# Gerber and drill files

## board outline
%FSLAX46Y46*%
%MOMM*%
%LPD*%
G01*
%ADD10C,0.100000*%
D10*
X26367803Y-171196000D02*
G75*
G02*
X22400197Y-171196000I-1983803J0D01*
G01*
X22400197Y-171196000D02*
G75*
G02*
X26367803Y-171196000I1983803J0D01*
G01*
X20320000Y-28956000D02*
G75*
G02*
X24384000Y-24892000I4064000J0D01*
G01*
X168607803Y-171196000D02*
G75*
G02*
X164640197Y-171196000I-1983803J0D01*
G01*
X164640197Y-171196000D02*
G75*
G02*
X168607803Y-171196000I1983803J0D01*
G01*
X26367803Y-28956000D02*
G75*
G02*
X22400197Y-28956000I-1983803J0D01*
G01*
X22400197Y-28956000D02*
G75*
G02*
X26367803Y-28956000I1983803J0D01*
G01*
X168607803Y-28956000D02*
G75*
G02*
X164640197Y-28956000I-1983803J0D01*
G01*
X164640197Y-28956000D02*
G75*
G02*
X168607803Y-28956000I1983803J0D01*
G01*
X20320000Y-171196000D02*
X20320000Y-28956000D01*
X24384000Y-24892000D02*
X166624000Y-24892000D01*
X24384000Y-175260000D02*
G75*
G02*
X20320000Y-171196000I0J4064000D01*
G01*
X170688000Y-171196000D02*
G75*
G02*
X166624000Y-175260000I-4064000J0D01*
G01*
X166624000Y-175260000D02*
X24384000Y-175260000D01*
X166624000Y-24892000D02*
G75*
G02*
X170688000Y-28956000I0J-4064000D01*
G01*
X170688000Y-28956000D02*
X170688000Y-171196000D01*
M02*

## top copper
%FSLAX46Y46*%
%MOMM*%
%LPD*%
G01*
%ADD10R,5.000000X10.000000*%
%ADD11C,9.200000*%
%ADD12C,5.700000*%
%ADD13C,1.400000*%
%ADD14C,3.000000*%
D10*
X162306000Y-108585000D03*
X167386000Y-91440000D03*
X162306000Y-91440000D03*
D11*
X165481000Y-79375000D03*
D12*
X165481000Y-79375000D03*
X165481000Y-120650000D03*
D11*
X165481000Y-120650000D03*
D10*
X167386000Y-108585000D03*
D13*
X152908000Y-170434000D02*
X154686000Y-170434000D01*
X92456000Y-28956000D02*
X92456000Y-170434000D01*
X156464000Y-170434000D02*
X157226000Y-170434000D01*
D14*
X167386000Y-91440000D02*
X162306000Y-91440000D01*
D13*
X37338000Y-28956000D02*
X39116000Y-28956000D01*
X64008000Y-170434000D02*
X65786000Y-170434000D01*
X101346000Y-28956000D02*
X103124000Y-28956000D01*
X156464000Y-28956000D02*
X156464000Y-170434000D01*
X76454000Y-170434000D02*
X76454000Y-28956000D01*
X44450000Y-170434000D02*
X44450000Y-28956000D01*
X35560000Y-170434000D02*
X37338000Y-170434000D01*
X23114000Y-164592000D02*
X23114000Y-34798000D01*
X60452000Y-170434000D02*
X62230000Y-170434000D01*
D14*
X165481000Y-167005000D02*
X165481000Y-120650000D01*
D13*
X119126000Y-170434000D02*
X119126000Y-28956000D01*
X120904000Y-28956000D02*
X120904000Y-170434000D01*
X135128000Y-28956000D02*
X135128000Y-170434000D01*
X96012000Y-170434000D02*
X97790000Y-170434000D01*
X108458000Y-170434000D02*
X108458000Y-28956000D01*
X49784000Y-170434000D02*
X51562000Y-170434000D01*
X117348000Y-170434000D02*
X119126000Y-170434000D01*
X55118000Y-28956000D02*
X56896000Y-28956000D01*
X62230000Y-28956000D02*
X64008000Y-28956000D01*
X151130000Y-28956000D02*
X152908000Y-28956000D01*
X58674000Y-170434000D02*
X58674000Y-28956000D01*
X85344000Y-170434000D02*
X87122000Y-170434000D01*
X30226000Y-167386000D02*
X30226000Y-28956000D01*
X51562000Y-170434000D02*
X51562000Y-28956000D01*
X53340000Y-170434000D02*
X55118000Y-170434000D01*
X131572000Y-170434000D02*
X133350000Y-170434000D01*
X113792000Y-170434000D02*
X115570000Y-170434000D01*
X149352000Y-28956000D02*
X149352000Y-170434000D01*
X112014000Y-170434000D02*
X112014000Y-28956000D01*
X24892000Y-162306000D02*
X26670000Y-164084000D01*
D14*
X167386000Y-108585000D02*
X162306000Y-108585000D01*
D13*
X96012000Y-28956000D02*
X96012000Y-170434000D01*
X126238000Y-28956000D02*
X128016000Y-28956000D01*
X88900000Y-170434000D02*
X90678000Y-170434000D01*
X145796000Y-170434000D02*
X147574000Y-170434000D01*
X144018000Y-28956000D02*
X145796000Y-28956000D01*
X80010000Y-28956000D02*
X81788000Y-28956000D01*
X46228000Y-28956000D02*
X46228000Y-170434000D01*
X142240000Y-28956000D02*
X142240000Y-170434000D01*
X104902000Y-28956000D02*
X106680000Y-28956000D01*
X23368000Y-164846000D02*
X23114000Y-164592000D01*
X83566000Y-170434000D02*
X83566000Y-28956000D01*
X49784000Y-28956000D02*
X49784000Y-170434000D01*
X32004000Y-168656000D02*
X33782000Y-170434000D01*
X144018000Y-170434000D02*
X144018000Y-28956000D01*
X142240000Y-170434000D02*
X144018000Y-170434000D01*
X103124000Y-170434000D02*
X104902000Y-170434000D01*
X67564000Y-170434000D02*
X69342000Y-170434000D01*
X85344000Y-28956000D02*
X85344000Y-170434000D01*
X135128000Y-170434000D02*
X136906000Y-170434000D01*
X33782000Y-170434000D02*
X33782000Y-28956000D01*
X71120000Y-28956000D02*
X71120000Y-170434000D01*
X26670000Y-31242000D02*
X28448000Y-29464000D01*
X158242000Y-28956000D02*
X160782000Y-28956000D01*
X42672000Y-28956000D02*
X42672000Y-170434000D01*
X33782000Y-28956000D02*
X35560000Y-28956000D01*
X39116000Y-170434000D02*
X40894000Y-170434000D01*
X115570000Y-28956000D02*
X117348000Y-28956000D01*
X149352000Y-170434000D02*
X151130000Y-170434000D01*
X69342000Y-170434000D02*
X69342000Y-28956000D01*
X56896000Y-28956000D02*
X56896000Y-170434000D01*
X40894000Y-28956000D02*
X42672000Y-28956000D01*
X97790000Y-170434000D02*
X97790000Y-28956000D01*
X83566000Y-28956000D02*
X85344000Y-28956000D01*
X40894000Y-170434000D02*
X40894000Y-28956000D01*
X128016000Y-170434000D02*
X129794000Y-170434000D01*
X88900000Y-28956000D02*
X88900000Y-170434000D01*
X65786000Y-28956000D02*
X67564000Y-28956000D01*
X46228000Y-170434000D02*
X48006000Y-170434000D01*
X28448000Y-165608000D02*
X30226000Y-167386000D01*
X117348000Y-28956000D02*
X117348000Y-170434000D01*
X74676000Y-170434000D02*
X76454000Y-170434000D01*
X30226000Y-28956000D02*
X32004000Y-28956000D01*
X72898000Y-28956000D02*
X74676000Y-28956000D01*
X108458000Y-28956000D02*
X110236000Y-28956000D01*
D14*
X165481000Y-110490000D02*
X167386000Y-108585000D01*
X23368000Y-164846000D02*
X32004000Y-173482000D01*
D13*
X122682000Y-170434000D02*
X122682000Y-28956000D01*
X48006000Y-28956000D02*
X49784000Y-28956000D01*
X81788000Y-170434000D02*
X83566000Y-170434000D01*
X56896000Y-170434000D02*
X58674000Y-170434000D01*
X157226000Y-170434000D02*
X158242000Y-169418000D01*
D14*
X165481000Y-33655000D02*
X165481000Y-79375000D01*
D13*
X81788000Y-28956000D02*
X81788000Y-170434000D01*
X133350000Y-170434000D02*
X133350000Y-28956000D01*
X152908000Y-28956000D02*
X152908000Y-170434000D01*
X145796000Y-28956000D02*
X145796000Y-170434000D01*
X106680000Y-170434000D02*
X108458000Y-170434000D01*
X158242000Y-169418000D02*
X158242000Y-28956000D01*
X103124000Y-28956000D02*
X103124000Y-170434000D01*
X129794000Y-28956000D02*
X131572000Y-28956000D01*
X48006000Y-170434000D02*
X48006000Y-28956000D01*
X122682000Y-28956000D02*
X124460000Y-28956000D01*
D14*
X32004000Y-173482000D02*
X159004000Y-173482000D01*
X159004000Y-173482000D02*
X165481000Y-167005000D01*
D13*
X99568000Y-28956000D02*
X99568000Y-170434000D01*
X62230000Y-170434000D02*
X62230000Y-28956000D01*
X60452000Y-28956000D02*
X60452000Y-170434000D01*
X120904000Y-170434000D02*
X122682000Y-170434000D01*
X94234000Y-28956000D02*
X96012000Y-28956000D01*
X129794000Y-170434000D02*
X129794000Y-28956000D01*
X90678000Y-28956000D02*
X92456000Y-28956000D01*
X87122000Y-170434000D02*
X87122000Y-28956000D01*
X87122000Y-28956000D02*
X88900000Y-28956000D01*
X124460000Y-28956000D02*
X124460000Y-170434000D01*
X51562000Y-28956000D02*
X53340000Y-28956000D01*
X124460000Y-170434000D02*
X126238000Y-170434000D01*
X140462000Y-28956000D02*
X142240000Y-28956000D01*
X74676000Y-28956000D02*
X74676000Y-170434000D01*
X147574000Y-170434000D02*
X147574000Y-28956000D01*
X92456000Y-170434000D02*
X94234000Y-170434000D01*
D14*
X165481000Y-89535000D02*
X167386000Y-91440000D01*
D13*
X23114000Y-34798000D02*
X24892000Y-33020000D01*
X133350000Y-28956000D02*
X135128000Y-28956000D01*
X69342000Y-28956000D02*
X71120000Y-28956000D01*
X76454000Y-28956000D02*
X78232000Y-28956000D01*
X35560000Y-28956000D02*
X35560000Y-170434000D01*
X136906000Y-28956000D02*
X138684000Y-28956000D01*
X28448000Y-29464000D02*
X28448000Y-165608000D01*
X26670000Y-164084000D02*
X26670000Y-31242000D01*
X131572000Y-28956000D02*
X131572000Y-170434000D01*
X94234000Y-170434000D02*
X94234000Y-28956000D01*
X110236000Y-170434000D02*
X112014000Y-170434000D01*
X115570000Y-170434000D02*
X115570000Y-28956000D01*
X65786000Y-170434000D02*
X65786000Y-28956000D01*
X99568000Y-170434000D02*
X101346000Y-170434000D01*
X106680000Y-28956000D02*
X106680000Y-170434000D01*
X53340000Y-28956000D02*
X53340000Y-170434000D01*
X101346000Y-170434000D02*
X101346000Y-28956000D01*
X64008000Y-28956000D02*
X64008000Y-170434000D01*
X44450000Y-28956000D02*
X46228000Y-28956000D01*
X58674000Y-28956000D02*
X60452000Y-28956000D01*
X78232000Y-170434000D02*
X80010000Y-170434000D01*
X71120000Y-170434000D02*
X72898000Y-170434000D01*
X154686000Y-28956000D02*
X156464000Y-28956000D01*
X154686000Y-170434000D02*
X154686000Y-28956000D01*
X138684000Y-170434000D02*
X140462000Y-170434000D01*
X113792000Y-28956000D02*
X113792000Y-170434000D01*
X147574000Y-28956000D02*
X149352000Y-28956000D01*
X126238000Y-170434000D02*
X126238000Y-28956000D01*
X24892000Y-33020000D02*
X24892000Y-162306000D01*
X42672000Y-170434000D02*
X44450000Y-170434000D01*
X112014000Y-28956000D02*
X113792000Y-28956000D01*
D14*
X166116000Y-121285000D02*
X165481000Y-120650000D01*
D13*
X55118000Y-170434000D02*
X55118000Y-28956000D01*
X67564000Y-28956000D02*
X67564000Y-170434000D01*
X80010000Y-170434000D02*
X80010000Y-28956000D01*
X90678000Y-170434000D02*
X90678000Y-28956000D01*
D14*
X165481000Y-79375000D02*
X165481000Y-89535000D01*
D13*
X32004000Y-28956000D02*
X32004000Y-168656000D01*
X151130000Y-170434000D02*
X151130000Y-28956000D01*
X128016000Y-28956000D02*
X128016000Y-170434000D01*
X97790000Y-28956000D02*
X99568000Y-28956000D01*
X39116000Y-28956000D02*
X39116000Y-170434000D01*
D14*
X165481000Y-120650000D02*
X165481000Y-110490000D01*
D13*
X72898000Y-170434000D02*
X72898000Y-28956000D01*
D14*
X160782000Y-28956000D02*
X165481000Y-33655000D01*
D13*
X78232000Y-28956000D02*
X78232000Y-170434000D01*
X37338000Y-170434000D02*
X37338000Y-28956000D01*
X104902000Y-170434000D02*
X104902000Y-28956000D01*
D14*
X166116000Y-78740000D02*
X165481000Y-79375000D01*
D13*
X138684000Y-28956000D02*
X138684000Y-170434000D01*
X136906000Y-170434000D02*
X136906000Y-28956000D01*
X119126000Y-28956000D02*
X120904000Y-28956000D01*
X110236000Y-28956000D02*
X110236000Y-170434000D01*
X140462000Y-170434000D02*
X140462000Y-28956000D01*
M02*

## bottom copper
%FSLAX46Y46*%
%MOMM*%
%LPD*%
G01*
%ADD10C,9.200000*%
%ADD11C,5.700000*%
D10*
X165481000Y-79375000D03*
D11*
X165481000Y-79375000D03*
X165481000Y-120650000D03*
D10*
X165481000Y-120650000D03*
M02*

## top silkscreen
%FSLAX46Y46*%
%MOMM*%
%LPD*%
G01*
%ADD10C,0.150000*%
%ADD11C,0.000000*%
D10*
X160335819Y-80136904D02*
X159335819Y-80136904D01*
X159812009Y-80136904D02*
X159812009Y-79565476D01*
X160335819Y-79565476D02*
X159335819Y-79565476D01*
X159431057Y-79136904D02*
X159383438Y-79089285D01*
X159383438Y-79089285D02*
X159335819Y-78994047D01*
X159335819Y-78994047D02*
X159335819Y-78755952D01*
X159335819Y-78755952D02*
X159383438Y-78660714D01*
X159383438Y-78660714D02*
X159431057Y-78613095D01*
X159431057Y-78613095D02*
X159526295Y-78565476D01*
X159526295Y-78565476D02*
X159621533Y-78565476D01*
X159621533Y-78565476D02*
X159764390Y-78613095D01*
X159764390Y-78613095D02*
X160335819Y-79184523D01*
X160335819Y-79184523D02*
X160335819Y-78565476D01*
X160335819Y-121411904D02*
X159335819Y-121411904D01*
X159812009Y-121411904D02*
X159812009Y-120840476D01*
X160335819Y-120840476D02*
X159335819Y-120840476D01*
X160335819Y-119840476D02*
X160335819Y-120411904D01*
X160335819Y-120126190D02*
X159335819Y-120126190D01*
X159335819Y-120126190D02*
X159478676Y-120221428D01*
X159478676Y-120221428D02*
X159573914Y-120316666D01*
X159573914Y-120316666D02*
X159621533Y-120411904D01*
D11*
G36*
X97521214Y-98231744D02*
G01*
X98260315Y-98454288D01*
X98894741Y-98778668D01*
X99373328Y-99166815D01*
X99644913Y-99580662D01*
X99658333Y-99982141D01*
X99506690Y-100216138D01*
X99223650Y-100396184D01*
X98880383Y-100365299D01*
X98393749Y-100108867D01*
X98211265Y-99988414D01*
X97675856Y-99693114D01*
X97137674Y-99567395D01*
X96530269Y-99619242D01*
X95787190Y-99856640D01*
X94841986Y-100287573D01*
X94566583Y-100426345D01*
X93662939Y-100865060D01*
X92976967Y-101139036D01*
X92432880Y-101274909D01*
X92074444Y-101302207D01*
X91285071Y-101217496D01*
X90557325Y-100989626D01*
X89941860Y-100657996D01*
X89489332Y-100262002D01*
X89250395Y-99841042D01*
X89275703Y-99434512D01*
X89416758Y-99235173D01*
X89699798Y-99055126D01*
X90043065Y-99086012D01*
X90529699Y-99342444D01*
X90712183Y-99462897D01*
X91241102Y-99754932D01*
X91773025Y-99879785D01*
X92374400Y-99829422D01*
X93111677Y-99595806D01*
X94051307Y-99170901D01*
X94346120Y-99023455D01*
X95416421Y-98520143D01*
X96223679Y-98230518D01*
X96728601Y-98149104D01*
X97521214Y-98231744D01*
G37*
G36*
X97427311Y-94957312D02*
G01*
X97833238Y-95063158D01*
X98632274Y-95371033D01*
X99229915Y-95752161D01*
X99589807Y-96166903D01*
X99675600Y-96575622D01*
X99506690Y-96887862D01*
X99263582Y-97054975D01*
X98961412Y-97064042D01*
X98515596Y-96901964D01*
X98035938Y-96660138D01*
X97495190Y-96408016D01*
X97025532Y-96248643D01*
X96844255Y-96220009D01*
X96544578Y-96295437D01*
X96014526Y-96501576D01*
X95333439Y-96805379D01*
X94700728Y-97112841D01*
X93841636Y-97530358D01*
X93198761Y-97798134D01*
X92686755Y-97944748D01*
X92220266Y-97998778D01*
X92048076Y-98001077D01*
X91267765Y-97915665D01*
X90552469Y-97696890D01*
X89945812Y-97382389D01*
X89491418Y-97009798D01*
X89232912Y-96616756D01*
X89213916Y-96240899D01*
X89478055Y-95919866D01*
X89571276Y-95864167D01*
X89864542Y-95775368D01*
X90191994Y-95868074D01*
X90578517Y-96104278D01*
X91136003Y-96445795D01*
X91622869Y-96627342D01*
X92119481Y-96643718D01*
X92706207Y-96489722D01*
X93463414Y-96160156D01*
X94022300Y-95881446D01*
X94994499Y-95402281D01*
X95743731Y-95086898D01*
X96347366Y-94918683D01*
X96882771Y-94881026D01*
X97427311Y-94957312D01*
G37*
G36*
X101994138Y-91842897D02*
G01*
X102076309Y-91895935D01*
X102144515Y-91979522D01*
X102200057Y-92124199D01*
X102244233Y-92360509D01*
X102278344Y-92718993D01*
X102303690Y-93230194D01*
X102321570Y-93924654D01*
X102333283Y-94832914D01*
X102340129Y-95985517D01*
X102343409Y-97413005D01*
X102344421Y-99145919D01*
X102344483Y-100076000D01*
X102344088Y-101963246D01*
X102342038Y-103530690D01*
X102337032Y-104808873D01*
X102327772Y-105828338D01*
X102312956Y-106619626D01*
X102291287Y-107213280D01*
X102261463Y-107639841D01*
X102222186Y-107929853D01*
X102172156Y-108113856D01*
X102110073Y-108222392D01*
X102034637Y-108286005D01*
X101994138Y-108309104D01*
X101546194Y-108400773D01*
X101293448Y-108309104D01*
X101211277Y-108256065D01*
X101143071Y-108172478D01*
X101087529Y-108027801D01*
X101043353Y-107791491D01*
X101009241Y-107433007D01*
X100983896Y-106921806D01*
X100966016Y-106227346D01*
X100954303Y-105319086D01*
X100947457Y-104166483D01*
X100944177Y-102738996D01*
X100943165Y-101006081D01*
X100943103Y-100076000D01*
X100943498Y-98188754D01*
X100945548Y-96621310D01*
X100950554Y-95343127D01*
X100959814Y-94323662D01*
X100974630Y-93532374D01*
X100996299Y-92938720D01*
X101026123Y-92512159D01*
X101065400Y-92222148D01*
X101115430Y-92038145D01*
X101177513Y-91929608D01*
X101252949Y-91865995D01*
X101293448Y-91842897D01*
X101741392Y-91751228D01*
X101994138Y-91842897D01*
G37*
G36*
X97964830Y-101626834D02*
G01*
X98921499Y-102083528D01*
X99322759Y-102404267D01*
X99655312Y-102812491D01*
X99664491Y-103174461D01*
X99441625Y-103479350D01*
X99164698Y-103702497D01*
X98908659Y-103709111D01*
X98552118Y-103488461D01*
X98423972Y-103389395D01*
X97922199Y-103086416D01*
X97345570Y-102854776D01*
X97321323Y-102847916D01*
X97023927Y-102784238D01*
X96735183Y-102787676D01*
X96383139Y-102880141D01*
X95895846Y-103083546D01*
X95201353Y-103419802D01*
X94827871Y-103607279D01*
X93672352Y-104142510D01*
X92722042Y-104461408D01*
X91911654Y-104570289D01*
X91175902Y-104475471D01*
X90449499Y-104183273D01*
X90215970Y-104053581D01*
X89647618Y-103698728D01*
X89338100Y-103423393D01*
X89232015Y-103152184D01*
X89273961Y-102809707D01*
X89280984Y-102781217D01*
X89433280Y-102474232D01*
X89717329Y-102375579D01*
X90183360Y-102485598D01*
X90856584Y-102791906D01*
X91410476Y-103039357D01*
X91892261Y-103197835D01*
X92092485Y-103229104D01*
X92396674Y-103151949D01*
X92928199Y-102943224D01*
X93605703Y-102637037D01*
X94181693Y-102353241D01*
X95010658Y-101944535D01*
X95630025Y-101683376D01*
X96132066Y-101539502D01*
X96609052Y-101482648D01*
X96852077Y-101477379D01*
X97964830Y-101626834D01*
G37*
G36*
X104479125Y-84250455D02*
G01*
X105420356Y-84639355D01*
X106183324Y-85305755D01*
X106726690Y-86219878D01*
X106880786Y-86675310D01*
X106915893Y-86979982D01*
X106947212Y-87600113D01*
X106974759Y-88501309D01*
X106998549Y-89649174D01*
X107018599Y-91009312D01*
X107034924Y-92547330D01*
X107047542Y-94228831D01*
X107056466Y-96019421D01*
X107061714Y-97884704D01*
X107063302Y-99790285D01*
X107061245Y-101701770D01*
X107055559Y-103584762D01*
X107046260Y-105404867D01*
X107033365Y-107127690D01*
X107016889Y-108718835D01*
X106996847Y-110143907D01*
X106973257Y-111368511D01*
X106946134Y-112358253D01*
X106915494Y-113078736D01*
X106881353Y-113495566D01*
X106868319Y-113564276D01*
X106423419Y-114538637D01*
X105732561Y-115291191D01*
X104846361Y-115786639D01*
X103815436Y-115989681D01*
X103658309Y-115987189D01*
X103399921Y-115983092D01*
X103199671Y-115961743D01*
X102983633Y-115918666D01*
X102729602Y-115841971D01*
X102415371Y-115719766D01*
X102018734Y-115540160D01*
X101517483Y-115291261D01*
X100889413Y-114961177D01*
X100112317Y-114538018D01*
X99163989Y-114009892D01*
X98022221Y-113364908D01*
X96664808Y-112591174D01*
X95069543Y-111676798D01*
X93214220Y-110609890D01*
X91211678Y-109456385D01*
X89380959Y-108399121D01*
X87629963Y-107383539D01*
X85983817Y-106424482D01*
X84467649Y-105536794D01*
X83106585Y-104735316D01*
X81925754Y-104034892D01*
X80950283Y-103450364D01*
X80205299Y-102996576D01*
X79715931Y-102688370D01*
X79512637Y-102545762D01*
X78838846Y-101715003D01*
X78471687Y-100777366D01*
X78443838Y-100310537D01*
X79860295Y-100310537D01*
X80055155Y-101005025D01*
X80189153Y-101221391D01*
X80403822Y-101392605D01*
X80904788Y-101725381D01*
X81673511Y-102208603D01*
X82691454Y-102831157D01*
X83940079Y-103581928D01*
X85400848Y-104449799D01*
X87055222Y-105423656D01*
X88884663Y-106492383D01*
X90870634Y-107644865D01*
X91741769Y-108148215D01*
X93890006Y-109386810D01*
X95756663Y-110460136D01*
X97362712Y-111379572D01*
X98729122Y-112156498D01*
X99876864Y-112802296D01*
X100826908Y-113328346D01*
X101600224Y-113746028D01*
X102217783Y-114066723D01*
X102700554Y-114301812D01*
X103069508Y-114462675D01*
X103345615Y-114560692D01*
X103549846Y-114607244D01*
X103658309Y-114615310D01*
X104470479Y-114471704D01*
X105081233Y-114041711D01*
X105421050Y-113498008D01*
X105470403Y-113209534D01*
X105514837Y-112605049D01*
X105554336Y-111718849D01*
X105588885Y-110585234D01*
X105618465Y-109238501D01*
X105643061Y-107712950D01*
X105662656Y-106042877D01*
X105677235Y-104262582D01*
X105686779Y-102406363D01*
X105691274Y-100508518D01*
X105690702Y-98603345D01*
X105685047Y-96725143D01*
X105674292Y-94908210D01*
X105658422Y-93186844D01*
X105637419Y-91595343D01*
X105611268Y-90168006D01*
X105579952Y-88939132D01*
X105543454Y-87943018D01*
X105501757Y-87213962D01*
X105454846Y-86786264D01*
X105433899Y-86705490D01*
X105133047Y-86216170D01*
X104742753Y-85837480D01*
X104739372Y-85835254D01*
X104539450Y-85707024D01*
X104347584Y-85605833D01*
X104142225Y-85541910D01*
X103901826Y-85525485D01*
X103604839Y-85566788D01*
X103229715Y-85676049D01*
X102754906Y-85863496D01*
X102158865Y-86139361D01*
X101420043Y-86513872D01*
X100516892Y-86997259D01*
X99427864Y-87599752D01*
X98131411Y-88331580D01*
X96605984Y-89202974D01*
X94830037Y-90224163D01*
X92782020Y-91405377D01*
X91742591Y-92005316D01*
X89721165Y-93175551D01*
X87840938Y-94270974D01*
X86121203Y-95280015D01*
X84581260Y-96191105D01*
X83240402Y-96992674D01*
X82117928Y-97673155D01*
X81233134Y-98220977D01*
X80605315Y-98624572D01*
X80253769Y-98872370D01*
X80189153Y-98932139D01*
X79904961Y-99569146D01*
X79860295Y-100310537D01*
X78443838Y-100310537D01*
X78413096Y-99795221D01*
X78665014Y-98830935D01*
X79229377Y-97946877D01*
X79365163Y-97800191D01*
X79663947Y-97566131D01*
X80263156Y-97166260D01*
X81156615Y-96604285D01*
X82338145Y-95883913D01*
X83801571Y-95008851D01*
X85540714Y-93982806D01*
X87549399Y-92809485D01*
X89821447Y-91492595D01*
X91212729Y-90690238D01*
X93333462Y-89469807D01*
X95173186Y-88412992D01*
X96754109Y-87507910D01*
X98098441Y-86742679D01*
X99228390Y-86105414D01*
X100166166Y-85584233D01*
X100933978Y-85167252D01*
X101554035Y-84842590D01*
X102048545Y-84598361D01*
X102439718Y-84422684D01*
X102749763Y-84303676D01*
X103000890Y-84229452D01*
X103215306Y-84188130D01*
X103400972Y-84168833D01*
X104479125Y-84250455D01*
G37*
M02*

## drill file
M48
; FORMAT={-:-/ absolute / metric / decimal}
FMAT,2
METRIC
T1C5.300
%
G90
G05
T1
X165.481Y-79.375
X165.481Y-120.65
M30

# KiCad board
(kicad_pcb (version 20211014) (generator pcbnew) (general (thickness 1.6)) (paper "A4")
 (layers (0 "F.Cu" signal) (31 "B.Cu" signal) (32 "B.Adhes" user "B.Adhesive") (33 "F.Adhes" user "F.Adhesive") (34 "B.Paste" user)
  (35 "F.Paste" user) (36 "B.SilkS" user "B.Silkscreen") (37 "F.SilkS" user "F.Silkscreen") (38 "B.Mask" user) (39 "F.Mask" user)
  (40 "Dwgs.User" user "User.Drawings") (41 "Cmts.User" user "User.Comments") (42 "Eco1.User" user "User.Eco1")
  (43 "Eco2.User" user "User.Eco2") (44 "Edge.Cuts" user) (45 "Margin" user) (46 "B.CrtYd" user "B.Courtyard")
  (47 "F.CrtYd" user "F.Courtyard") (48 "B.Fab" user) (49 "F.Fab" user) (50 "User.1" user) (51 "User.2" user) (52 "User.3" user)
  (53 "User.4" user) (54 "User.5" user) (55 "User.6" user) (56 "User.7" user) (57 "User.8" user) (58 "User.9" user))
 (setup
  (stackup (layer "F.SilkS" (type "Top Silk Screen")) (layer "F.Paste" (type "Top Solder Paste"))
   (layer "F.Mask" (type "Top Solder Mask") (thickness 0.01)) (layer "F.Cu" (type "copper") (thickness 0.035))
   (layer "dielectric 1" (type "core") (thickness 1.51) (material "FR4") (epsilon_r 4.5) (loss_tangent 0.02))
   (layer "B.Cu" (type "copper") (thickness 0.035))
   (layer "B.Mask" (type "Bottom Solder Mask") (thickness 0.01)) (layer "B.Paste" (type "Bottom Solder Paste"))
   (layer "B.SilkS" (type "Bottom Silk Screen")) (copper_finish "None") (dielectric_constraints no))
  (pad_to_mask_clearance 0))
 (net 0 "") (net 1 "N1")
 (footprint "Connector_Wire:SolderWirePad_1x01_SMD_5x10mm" (layer "F.Cu") (at 162.306 108.585)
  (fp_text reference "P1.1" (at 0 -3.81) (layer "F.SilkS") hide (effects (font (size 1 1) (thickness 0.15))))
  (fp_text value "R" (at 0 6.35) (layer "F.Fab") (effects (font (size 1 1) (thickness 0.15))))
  (pad "1" smd rect (at 0 0) (size 5 10) (layers "F.Cu" "F.Paste" "F.Mask") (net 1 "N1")))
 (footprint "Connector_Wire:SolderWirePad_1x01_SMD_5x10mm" (layer "F.Cu") (at 167.386 91.44)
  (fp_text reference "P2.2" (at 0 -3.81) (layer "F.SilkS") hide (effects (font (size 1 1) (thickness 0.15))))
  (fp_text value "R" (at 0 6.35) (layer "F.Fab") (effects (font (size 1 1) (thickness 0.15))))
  (pad "1" smd rect (at 0 0) (size 5 10) (layers "F.Cu" "F.Paste" "F.Mask") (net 1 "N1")))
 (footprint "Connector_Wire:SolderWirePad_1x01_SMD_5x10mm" (layer "F.Cu") (at 162.306 91.44)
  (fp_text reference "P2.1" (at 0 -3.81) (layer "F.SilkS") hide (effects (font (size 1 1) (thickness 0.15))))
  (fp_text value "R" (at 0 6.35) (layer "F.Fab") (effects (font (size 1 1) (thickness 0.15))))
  (pad "1" smd rect (at 0 0) (size 5 10) (layers "F.Cu" "F.Paste" "F.Mask") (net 1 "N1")))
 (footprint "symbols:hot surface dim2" (layer "F.Cu") (at 92.71 100.076 90)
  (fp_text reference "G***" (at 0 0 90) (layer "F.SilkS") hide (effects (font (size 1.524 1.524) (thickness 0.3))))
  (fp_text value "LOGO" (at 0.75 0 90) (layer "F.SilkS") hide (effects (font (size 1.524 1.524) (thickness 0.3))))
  (fp_poly
   (pts (xy 0.641488 -3.434297) (xy 0.840827 -3.293242) (xy 1.020874 -3.010202) (xy 0.989988 -2.666935) (xy 0.733556 -2.180301)
    (xy 0.613103 -1.997817) (xy 0.321068 -1.468898) (xy 0.196215 -0.936975) (xy 0.246578 -0.3356) (xy 0.480194 0.401677)
    (xy 0.905099 1.341307) (xy 1.052545 1.63612) (xy 1.555857 2.706421) (xy 1.845482 3.513679) (xy 1.926896 4.018601) (xy 1.844256 4.811214)
    (xy 1.621712 5.550315) (xy 1.297332 6.184741) (xy 0.909185 6.663328) (xy 0.495338 6.934913) (xy 0.093859 6.948333)
    (xy -0.140138 6.79669) (xy -0.320184 6.51365) (xy -0.289299 6.170383) (xy -0.032867 5.683749) (xy 0.087586 5.501265)
    (xy 0.382886 4.965856) (xy 0.508605 4.427674) (xy 0.456758 3.820269) (xy 0.21936 3.07719) (xy -0.211573 2.131986)
    (xy -0.350345 1.856583) (xy -0.78906 0.952939) (xy -1.063036 0.266967) (xy -1.198909 -0.27712) (xy -1.226207 -0.635556)
    (xy -1.141496 -1.424929) (xy -0.913626 -2.152675) (xy -0.581996 -2.76814) (xy -0.186002 -3.220668) (xy 0.234958 -3.459605))
   (layer "F.SilkS") (width 0) (fill solid))
  (fp_poly
   (pts (xy 4.156134 -3.231945) (xy 4.211833 -3.138724) (xy 4.300632 -2.845458) (xy 4.207926 -2.518006) (xy 3.971722 -2.131483)
    (xy 3.630205 -1.573997) (xy 3.448658 -1.087131) (xy 3.432282 -0.590519) (xy 3.586278 -0.003793) (xy 3.915844 0.753414)
    (xy 4.194554 1.3123) (xy 4.673719 2.284499) (xy 4.989102 3.033731) (xy 5.157317 3.637366) (xy 5.194974 4.172771) (xy 5.118688 4.717311)
    (xy 5.012842 5.123238) (xy 4.704967 5.922274) (xy 4.323839 6.519915) (xy 3.909097 6.879807) (xy 3.500378 6.9656) (xy 3.188138 6.79669)
    (xy 3.021025 6.553582) (xy 3.011958 6.251412) (xy 3.174036 5.805596) (xy 3.415862 5.325938) (xy 3.667984 4.78519) (xy 3.827357 4.315532)
    (xy 3.855991 4.134255) (xy 3.780563 3.834578) (xy 3.574424 3.304526) (xy 3.270621 2.623439) (xy 2.963159 1.990728)
    (xy 2.545642 1.131636) (xy 2.277866 0.488761) (xy 2.131252 -0.023245) (xy 2.077222 -0.489734) (xy 2.074923 -0.661924)
    (xy 2.160335 -1.442235) (xy 2.37911 -2.157531) (xy 2.693611 -2.764188) (xy 3.066202 -3.218582) (xy 3.459244 -3.477088)
    (xy 3.835101 -3.496084))
   (layer "F.SilkS") (width 0) (fill solid))
  (fp_poly
   (pts (xy 1.887246 8.233498) (xy 3.45469 8.235548) (xy 4.732873 8.240554) (xy 5.752338 8.249814) (xy 6.543626 8.26463)
    (xy 7.13728 8.286299) (xy 7.563841 8.316123) (xy 7.853852 8.3554) (xy 8.037855 8.40543) (xy 8.146392 8.467513) (xy 8.210005 8.542949)
    (xy 8.233103 8.583448) (xy 8.324772 9.031392) (xy 8.233103 9.284138) (xy 8.180065 9.366309) (xy 8.096478 9.434515)
    (xy 7.951801 9.490057) (xy 7.715491 9.534233) (xy 7.357007 9.568344) (xy 6.845806 9.59369) (xy 6.151346 9.61157) (xy 5.243086 9.623283)
    (xy 4.090483 9.630129) (xy 2.662995 9.633409) (xy 0.930081 9.634421) (xy 0 9.634483) (xy -1.887246 9.634088) (xy -3.45469 9.632038)
    (xy -4.732873 9.627032) (xy -5.752338 9.617772) (xy -6.543626 9.602956) (xy -7.13728 9.581287) (xy -7.563841 9.551463)
    (xy -7.853853 9.512186) (xy -8.037856 9.462156) (xy -8.146392 9.400073) (xy -8.210005 9.324637) (xy -8.233104 9.284138)
    (xy -8.324773 8.836194) (xy -8.233104 8.583448) (xy -8.180065 8.501277) (xy -8.096478 8.433071) (xy -7.951801 8.377529)
    (xy -7.715491 8.333353) (xy -7.357007 8.299241) (xy -6.845806 8.273896) (xy -6.151346 8.256016) (xy -5.243086 8.244303)
    (xy -4.090483 8.237457) (xy -2.662996 8.234177) (xy -0.930081 8.233165) (xy 0 8.233103))
   (layer "F.SilkS") (width 0) (fill solid))
  (fp_poly
   (pts (xy -2.733707 -3.436039) (xy -2.705217 -3.429016) (xy -2.398232 -3.27672) (xy -2.299579 -2.992671) (xy -2.409598 -2.52664)
    (xy -2.715906 -1.853416) (xy -2.963357 -1.299524) (xy -3.121835 -0.817739) (xy -3.153104 -0.617515) (xy -3.075949 -0.313326)
    (xy -2.867224 0.218199) (xy -2.561037 0.895703) (xy -2.277241 1.471693) (xy -1.868535 2.300658) (xy -1.607376 2.920025)
    (xy -1.463502 3.422066) (xy -1.406648 3.899052) (xy -1.401379 4.142077) (xy -1.550834 5.25483) (xy -2.007528 6.211499)
    (xy -2.328267 6.612759) (xy -2.736491 6.945312) (xy -3.098461 6.954491) (xy -3.40335 6.731625) (xy -3.626497 6.454698)
    (xy -3.633111 6.198659) (xy -3.412461 5.842118) (xy -3.313395 5.713972) (xy -3.010416 5.212199) (xy -2.778776 4.63557)
    (xy -2.771916 4.611323) (xy -2.708238 4.313927) (xy -2.711676 4.025183) (xy -2.804141 3.673139) (xy -3.007546 3.185846)
    (xy -3.343802 2.491353) (xy -3.531279 2.117871) (xy -4.06651 0.962352) (xy -4.385408 0.012042) (xy -4.494289 -0.798346)
    (xy -4.399471 -1.534098) (xy -4.107273 -2.260501) (xy -3.977581 -2.49403) (xy -3.622728 -3.062382) (xy -3.347393 -3.3719)
    (xy -3.076184 -3.477985))
   (layer "F.SilkS") (width 0) (fill solid))
  (fp_poly
   (pts (xy 1.245065 -14.044986) (xy 2.129123 -13.480623) (xy 2.275809 -13.344837) (xy 2.509869 -13.046053) (xy 2.90974 -12.446844)
    (xy 3.471715 -11.553385) (xy 4.192087 -10.371855) (xy 5.067149 -8.908429) (xy 6.093194 -7.169286) (xy 7.266515 -5.160601)
    (xy 8.583405 -2.888553) (xy 9.385762 -1.497271) (xy 10.606193 0.623462) (xy 11.663008 2.463186) (xy 12.56809 4.044109)
    (xy 13.333321 5.388441) (xy 13.970586 6.51839) (xy 14.491767 7.456166) (xy 14.908748 8.223978) (xy 15.23341 8.844035)
    (xy 15.477639 9.338545) (xy 15.653316 9.729718) (xy 15.772324 10.039763) (xy 15.846548 10.29089) (xy 15.88787 10.505306)
    (xy 15.907167 10.690972) (xy 15.825545 11.769125) (xy 15.436645 12.710356) (xy 14.770245 13.473324) (xy 13.856122 14.01669)
    (xy 13.40069 14.170786) (xy 13.096018 14.205893) (xy 12.475887 14.237212) (xy 11.574691 14.264759) (xy 10.426826 14.288549)
    (xy 9.066688 14.308599) (xy 7.52867 14.324924) (xy 5.847169 14.337542) (xy 4.056579 14.346466) (xy 2.191296 14.351714)
    (xy 0.285715 14.353302) (xy -1.62577 14.351245) (xy -3.508762 14.345559) (xy -5.328867 14.33626) (xy -7.05169 14.323365)
    (xy -8.642835 14.306889) (xy -10.067907 14.286847) (xy -11.292511 14.263257) (xy -12.282253 14.236134) (xy -13.002736 14.205494)
    (xy -13.419566 14.171353) (xy -13.488276 14.158319) (xy -14.462637 13.713419) (xy -15.215191 13.022561) (xy -15.710639 12.136361)
    (xy -15.913681 11.105436) (xy -15.911189 10.948309) (xy -14.53931 10.948309) (xy -14.395704 11.760479) (xy -13.965711 12.371233)
    (xy -13.422008 12.71105) (xy -13.133534 12.760403) (xy -12.529049 12.804837) (xy -11.642849 12.844336) (xy -10.509234 12.878885)
    (xy -9.162501 12.908465) (xy -7.63695 12.933061) (xy -5.966877 12.952656) (xy -4.186582 12.967235) (xy -2.330363 12.976779)
    (xy -0.432518 12.981274) (xy 1.472655 12.980702) (xy 3.350857 12.975047) (xy 5.16779 12.964292) (xy 6.889156 12.948422)
    (xy 8.480657 12.927419) (xy 9.907994 12.901268) (xy 11.136868 12.869952) (xy 12.132982 12.833454) (xy 12.862038 12.791757)
    (xy 13.289736 12.744846) (xy 13.37051 12.723899) (xy 13.85983 12.423047) (xy 14.23852 12.032753) (xy 14.240746 12.029372)
    (xy 14.368976 11.82945) (xy 14.470167 11.637584) (xy 14.53409 11.432225) (xy 14.550515 11.191826) (xy 14.509212 10.894839)
    (xy 14.399951 10.519715) (xy 14.212504 10.044906) (xy 13.936639 9.448865) (xy 13.562128 8.710043) (xy 13.078741 7.806892)
    (xy 12.476248 6.717864) (xy 11.74442 5.421411) (xy 10.873026 3.895984) (xy 9.851837 2.120037) (xy 8.670623 0.07202)
    (xy 8.070684 -0.967409) (xy 6.900449 -2.988835) (xy 5.805026 -4.869062) (xy 4.795985 -6.588797) (xy 3.884895 -8.12874)
    (xy 3.083326 -9.469598) (xy 2.402845 -10.592072) (xy 1.855023 -11.476866) (xy 1.451428 -12.104685) (xy 1.20363 -12.456231)
    (xy 1.143861 -12.520847) (xy 0.506854 -12.805039) (xy -0.234537 -12.849705) (xy -0.929025 -12.654845) (xy -1.145391 -12.520847)
    (xy -1.316605 -12.306178) (xy -1.649381 -11.805212) (xy -2.132603 -11.036489) (xy -2.755157 -10.018546) (xy -3.505928 -8.769921)
    (xy -4.373799 -7.309152) (xy -5.347656 -5.654778) (xy -6.416383 -3.825337) (xy -7.568865 -1.839366) (xy -8.072215 -0.968231)
    (xy -9.31081 1.180006) (xy -10.384136 3.046663) (xy -11.303572 4.652712) (xy -12.080498 6.019122) (xy -12.726296 7.166864)
    (xy -13.252346 8.116908) (xy -13.670028 8.890224) (xy -13.990723 9.507783) (xy -14.225812 9.990554) (xy -14.386675 10.359508)
    (xy -14.484692 10.635615) (xy -14.531244 10.839846) (xy -14.53931 10.948309) (xy -15.911189 10.948309) (xy -15.907092 10.689921)
    (xy -15.885743 10.489671) (xy -15.842666 10.273633) (xy -15.765971 10.019602) (xy -15.643766 9.705371) (xy -15.46416 9.308734)
    (xy -15.215261 8.807483) (xy -14.885177 8.179413) (xy -14.462018 7.402317) (xy -13.933892 6.453989) (xy -13.288908 5.312221)
    (xy -12.515174 3.954808) (xy -11.600798 2.359543) (xy -10.53389 0.50422) (xy -9.380385 -1.498322) (xy -8.323121 -3.329041)
    (xy -7.307539 -5.080037) (xy -6.348482 -6.726183) (xy -5.460794 -8.242351) (xy -4.659316 -9.603415) (xy -3.958892 -10.784246)
    (xy -3.374364 -11.759717) (xy -2.920576 -12.504701) (xy -2.61237 -12.994069) (xy -2.469762 -13.197363) (xy -1.639003 -13.871154)
    (xy -0.701366 -14.238313) (xy 0.280779 -14.296904))
   (layer "F.SilkS") (width 0) (fill solid)))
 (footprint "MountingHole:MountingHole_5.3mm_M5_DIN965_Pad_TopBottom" (layer "F.Cu") (at 165.481 79.375 90)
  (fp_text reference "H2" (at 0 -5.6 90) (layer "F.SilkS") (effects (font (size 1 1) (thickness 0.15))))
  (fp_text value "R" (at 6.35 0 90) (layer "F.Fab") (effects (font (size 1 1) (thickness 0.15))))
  (pad "1" connect circle (at 0 0 90) (size 9.2 9.2) (layers "B.Cu" "B.Mask") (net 1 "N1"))
  (pad "1" connect circle (at 0 0 90) (size 9.2 9.2) (layers "F.Cu" "F.Mask") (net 1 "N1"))
  (pad "1" thru_hole circle (at 0 0 90) (size 5.7 5.7) (drill 5.3) (layers *.Cu *.Mask) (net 1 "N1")))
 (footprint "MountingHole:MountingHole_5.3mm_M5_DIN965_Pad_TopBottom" (layer "F.Cu") (at 165.481 120.65 90)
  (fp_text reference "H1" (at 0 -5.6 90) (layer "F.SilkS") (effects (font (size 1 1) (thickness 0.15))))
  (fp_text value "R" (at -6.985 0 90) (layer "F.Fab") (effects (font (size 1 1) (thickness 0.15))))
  (pad "1" thru_hole circle (at 0 0 90) (size 5.7 5.7) (drill 5.3) (layers *.Cu *.Mask) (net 1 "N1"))
  (pad "1" connect circle (at 0 0 90) (size 9.2 9.2) (layers "F.Cu" "F.Mask") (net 1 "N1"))
  (pad "1" connect circle (at 0 0 90) (size 9.2 9.2) (layers "B.Cu" "B.Mask") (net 1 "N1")))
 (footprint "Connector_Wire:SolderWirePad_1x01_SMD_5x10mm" (layer "F.Cu") (at 167.386 108.585)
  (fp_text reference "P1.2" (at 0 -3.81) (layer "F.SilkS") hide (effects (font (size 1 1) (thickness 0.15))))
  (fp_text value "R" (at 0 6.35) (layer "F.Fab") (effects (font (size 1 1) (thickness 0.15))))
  (pad "1" smd rect (at 0 0) (size 5 10) (layers "F.Cu" "F.Paste" "F.Mask") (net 1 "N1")))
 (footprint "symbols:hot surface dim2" (layer "B.Cu") (at 92.71 100.076 -90)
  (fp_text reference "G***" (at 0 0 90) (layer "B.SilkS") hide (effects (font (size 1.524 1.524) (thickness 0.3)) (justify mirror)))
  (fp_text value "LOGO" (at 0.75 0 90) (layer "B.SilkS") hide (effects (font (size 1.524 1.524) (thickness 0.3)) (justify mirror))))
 (gr_circle (center 24.384 171.196) (end 22.86 169.926) (layer "Edge.Cuts") (width 0.1) (fill none))
 (gr_arc (start 20.32 28.956) (mid 21.510318 26.082318) (end 24.384 24.892) (layer "Edge.Cuts") (width 0.1))
 (gr_circle (center 166.624 171.196) (end 165.1 169.926) (layer "Edge.Cuts") (width 0.1) (fill none))
 (gr_circle (center 24.384 28.956) (end 22.86 27.686) (layer "Edge.Cuts") (width 0.1) (fill none))
 (gr_circle (center 166.624 28.956) (end 165.1 27.686) (layer "Edge.Cuts") (width 0.1) (fill none))
 (gr_line (start 20.32 171.196) (end 20.32 28.956) (layer "Edge.Cuts") (width 0.1))
 (gr_line (start 24.384 24.892) (end 166.624 24.892) (layer "Edge.Cuts") (width 0.1))
 (gr_arc (start 24.384 175.26) (mid 21.510318 174.069682) (end 20.32 171.196) (layer "Edge.Cuts") (width 0.1))
 (gr_arc (start 170.688 171.196) (mid 169.497682 174.069682) (end 166.624 175.26) (layer "Edge.Cuts") (width 0.1))
 (gr_line (start 166.624 175.26) (end 24.384 175.26) (layer "Edge.Cuts") (width 0.1))
 (gr_arc (start 166.624 24.892) (mid 169.497682 26.082318) (end 170.688 28.956) (layer "Edge.Cuts") (width 0.1))
 (gr_line (start 170.688 28.956) (end 170.688 171.196) (layer "Edge.Cuts") (width 0.1))
 (segment (start 152.908 170.434) (end 154.686 170.434) (width 1.4) (layer "F.Cu") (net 1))
 (segment (start 92.456 28.956) (end 92.456 170.434) (width 1.4) (layer "F.Cu") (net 1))
 (segment (start 156.464 170.434) (end 157.226 170.434) (width 1.4) (layer "F.Cu") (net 1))
 (segment (start 167.386 91.44) (end 162.306 91.44) (width 3) (layer "F.Cu") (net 1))
 (segment (start 37.338 28.956) (end 39.116 28.956) (width 1.4) (layer "F.Cu") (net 1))
 (segment (start 64.008 170.434) (end 65.786 170.434) (width 1.4) (layer "F.Cu") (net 1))
 (segment (start 101.346 28.956) (end 103.124 28.956) (width 1.4) (layer "F.Cu") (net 1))
 (segment (start 156.464 28.956) (end 156.464 170.434) (width 1.4) (layer "F.Cu") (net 1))
 (segment (start 76.454 170.434) (end 76.454 28.956) (width 1.4) (layer "F.Cu") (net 1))
 (segment (start 44.45 170.434) (end 44.45 28.956) (width 1.4) (layer "F.Cu") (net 1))
 (segment (start 35.56 170.434) (end 37.338 170.434) (width 1.4) (layer "F.Cu") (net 1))
 (segment (start 23.114 164.592) (end 23.114 34.798) (width 1.4) (layer "F.Cu") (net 1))
 (segment (start 60.452 170.434) (end 62.23 170.434) (width 1.4) (layer "F.Cu") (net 1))
 (segment (start 165.481 167.005) (end 165.481 120.65) (width 3) (layer "F.Cu") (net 1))
 (segment (start 119.126 170.434) (end 119.126 28.956) (width 1.4) (layer "F.Cu") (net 1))
 (segment (start 120.904 28.956) (end 120.904 170.434) (width 1.4) (layer "F.Cu") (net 1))
 (segment (start 135.128 28.956) (end 135.128 170.434) (width 1.4) (layer "F.Cu") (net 1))
 (segment (start 96.012 170.434) (end 97.79 170.434) (width 1.4) (layer "F.Cu") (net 1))
 (segment (start 108.458 170.434) (end 108.458 28.956) (width 1.4) (layer "F.Cu") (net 1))
 (segment (start 49.784 170.434) (end 51.562 170.434) (width 1.4) (layer "F.Cu") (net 1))
 (segment (start 117.348 170.434) (end 119.126 170.434) (width 1.4) (layer "F.Cu") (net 1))
 (segment (start 55.118 28.956) (end 56.896 28.956) (width 1.4) (layer "F.Cu") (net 1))
 (segment (start 62.23 28.956) (end 64.008 28.956) (width 1.4) (layer "F.Cu") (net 1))
 (segment (start 151.13 28.956) (end 152.908 28.956) (width 1.4) (layer "F.Cu") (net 1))
 (segment (start 58.674 170.434) (end 58.674 28.956) (width 1.4) (layer "F.Cu") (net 1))
 (segment (start 85.344 170.434) (end 87.122 170.434) (width 1.4) (layer "F.Cu") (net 1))
 (segment (start 30.226 167.386) (end 30.226 28.956) (width 1.4) (layer "F.Cu") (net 1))
 (segment (start 51.562 170.434) (end 51.562 28.956) (width 1.4) (layer "F.Cu") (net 1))
 (segment (start 53.34 170.434) (end 55.118 170.434) (width 1.4) (layer "F.Cu") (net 1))
 (segment (start 131.572 170.434) (end 133.35 170.434) (width 1.4) (layer "F.Cu") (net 1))
 (segment (start 113.792 170.434) (end 115.57 170.434) (width 1.4) (layer "F.Cu") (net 1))
 (segment (start 149.352 28.956) (end 149.352 170.434) (width 1.4) (layer "F.Cu") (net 1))
 (segment (start 112.014 170.434) (end 112.014 28.956) (width 1.4) (layer "F.Cu") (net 1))
 (segment (start 24.892 162.306) (end 26.67 164.084) (width 1.4) (layer "F.Cu") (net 1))
 (segment (start 167.386 108.585) (end 162.306 108.585) (width 3) (layer "F.Cu") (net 1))
 (segment (start 96.012 28.956) (end 96.012 170.434) (width 1.4) (layer "F.Cu") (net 1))
 (segment (start 126.238 28.956) (end 128.016 28.956) (width 1.4) (layer "F.Cu") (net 1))
 (segment (start 88.9 170.434) (end 90.678 170.434) (width 1.4) (layer "F.Cu") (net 1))
 (segment (start 145.796 170.434) (end 147.574 170.434) (width 1.4) (layer "F.Cu") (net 1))
 (segment (start 144.018 28.956) (end 145.796 28.956) (width 1.4) (layer "F.Cu") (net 1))
 (segment (start 80.01 28.956) (end 81.788 28.956) (width 1.4) (layer "F.Cu") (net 1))
 (segment (start 46.228 28.956) (end 46.228 170.434) (width 1.4) (layer "F.Cu") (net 1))
 (segment (start 142.24 28.956) (end 142.24 170.434) (width 1.4) (layer "F.Cu") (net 1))
 (segment (start 104.902 28.956) (end 106.68 28.956) (width 1.4) (layer "F.Cu") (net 1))
 (segment (start 23.368 164.846) (end 23.114 164.592) (width 1.4) (layer "F.Cu") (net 1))
 (segment (start 83.566 170.434) (end 83.566 28.956) (width 1.4) (layer "F.Cu") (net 1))
 (segment (start 49.784 28.956) (end 49.784 170.434) (width 1.4) (layer "F.Cu") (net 1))
 (segment (start 32.004 168.656) (end 33.782 170.434) (width 1.4) (layer "F.Cu") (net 1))
 (segment (start 144.018 170.434) (end 144.018 28.956) (width 1.4) (layer "F.Cu") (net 1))
 (segment (start 142.24 170.434) (end 144.018 170.434) (width 1.4) (layer "F.Cu") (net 1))
 (segment (start 103.124 170.434) (end 104.902 170.434) (width 1.4) (layer "F.Cu") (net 1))
 (segment (start 67.564 170.434) (end 69.342 170.434) (width 1.4) (layer "F.Cu") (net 1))
 (segment (start 85.344 28.956) (end 85.344 170.434) (width 1.4) (layer "F.Cu") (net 1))
 (segment (start 135.128 170.434) (end 136.906 170.434) (width 1.4) (layer "F.Cu") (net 1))
 (segment (start 33.782 170.434) (end 33.782 28.956) (width 1.4) (layer "F.Cu") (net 1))
 (segment (start 71.12 28.956) (end 71.12 170.434) (width 1.4) (layer "F.Cu") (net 1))
 (segment (start 26.67 31.242) (end 28.448 29.464) (width 1.4) (layer "F.Cu") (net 1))
 (segment (start 158.242 28.956) (end 160.782 28.956) (width 1.4) (layer "F.Cu") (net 1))
 (segment (start 42.672 28.956) (end 42.672 170.434) (width 1.4) (layer "F.Cu") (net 1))
 (segment (start 33.782 28.956) (end 35.56 28.956) (width 1.4) (layer "F.Cu") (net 1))
 (segment (start 39.116 170.434) (end 40.894 170.434) (width 1.4) (layer "F.Cu") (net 1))
 (segment (start 115.57 28.956) (end 117.348 28.956) (width 1.4) (layer "F.Cu") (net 1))
 (segment (start 149.352 170.434) (end 151.13 170.434) (width 1.4) (layer "F.Cu") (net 1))
 (segment (start 69.342 170.434) (end 69.342 28.956) (width 1.4) (layer "F.Cu") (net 1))
 (segment (start 56.896 28.956) (end 56.896 170.434) (width 1.4) (layer "F.Cu") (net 1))
 (segment (start 40.894 28.956) (end 42.672 28.956) (width 1.4) (layer "F.Cu") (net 1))
 (segment (start 97.79 170.434) (end 97.79 28.956) (width 1.4) (layer "F.Cu") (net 1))
 (segment (start 83.566 28.956) (end 85.344 28.956) (width 1.4) (layer "F.Cu") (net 1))
 (segment (start 40.894 170.434) (end 40.894 28.956) (width 1.4) (layer "F.Cu") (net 1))
 (segment (start 128.016 170.434) (end 129.794 170.434) (width 1.4) (layer "F.Cu") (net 1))
 (segment (start 88.9 28.956) (end 88.9 170.434) (width 1.4) (layer "F.Cu") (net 1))
 (segment (start 65.786 28.956) (end 67.564 28.956) (width 1.4) (layer "F.Cu") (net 1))
 (segment (start 46.228 170.434) (end 48.006 170.434) (width 1.4) (layer "F.Cu") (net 1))
 (segment (start 28.448 165.608) (end 30.226 167.386) (width 1.4) (layer "F.Cu") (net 1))
 (segment (start 117.348 28.956) (end 117.348 170.434) (width 1.4) (layer "F.Cu") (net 1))
 (segment (start 74.676 170.434) (end 76.454 170.434) (width 1.4) (layer "F.Cu") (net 1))
 (segment (start 30.226 28.956) (end 32.004 28.956) (width 1.4) (layer "F.Cu") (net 1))
 (segment (start 72.898 28.956) (end 74.676 28.956) (width 1.4) (layer "F.Cu") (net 1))
 (segment (start 108.458 28.956) (end 110.236 28.956) (width 1.4) (layer "F.Cu") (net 1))
 (segment (start 165.481 110.49) (end 167.386 108.585) (width 3) (layer "F.Cu") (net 1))
 (segment (start 23.368 164.846) (end 32.004 173.482) (width 3) (layer "F.Cu") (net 1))
 (segment (start 122.682 170.434) (end 122.682 28.956) (width 1.4) (layer "F.Cu") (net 1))
 (segment (start 48.006 28.956) (end 49.784 28.956) (width 1.4) (layer "F.Cu") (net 1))
 (segment (start 81.788 170.434) (end 83.566 170.434) (width 1.4) (layer "F.Cu") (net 1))
 (segment (start 56.896 170.434) (end 58.674 170.434) (width 1.4) (layer "F.Cu") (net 1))
 (segment (start 157.226 170.434) (end 158.242 169.418) (width 1.4) (layer "F.Cu") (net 1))
 (segment (start 165.481 33.655) (end 165.481 79.375) (width 3) (layer "F.Cu") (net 1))
 (segment (start 81.788 28.956) (end 81.788 170.434) (width 1.4) (layer "F.Cu") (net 1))
 (segment (start 133.35 170.434) (end 133.35 28.956) (width 1.4) (layer "F.Cu") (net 1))
 (segment (start 152.908 28.956) (end 152.908 170.434) (width 1.4) (layer "F.Cu") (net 1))
 (segment (start 145.796 28.956) (end 145.796 170.434) (width 1.4) (layer "F.Cu") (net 1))
 (segment (start 106.68 170.434) (end 108.458 170.434) (width 1.4) (layer "F.Cu") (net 1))
 (segment (start 158.242 169.418) (end 158.242 28.956) (width 1.4) (layer "F.Cu") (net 1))
 (segment (start 103.124 28.956) (end 103.124 170.434) (width 1.4) (layer "F.Cu") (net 1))
 (segment (start 129.794 28.956) (end 131.572 28.956) (width 1.4) (layer "F.Cu") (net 1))
 (segment (start 48.006 170.434) (end 48.006 28.956) (width 1.4) (layer "F.Cu") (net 1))
 (segment (start 122.682 28.956) (end 124.46 28.956) (width 1.4) (layer "F.Cu") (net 1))
 (segment (start 32.004 173.482) (end 159.004 173.482) (width 3) (layer "F.Cu") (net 1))
 (segment (start 159.004 173.482) (end 165.481 167.005) (width 3) (layer "F.Cu") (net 1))
 (segment (start 99.568 28.956) (end 99.568 170.434) (width 1.4) (layer "F.Cu") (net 1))
 (segment (start 62.23 170.434) (end 62.23 28.956) (width 1.4) (layer "F.Cu") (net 1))
 (segment (start 60.452 28.956) (end 60.452 170.434) (width 1.4) (layer "F.Cu") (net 1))
 (segment (start 120.904 170.434) (end 122.682 170.434) (width 1.4) (layer "F.Cu") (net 1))
 (segment (start 94.234 28.956) (end 96.012 28.956) (width 1.4) (layer "F.Cu") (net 1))
 (segment (start 129.794 170.434) (end 129.794 28.956) (width 1.4) (layer "F.Cu") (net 1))
 (segment (start 90.678 28.956) (end 92.456 28.956) (width 1.4) (layer "F.Cu") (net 1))
 (segment (start 87.122 170.434) (end 87.122 28.956) (width 1.4) (layer "F.Cu") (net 1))
 (segment (start 87.122 28.956) (end 88.9 28.956) (width 1.4) (layer "F.Cu") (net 1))
 (segment (start 124.46 28.956) (end 124.46 170.434) (width 1.4) (layer "F.Cu") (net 1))
 (segment (start 51.562 28.956) (end 53.34 28.956) (width 1.4) (layer "F.Cu") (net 1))
 (segment (start 124.46 170.434) (end 126.238 170.434) (width 1.4) (layer "F.Cu") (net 1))
 (segment (start 140.462 28.956) (end 142.24 28.956) (width 1.4) (layer "F.Cu") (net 1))
 (segment (start 74.676 28.956) (end 74.676 170.434) (width 1.4) (layer "F.Cu") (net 1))
 (segment (start 147.574 170.434) (end 147.574 28.956) (width 1.4) (layer "F.Cu") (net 1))
 (segment (start 92.456 170.434) (end 94.234 170.434) (width 1.4) (layer "F.Cu") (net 1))
 (segment (start 165.481 89.535) (end 167.386 91.44) (width 3) (layer "F.Cu") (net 1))
 (segment (start 23.114 34.798) (end 24.892 33.02) (width 1.4) (layer "F.Cu") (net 1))
 (segment (start 133.35 28.956) (end 135.128 28.956) (width 1.4) (layer "F.Cu") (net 1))
 (segment (start 69.342 28.956) (end 71.12 28.956) (width 1.4) (layer "F.Cu") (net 1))
 (segment (start 76.454 28.956) (end 78.232 28.956) (width 1.4) (layer "F.Cu") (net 1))
 (segment (start 35.56 28.956) (end 35.56 170.434) (width 1.4) (layer "F.Cu") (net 1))
 (segment (start 136.906 28.956) (end 138.684 28.956) (width 1.4) (layer "F.Cu") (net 1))
 (segment (start 28.448 29.464) (end 28.448 165.608) (width 1.4) (layer "F.Cu") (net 1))
 (segment (start 26.67 164.084) (end 26.67 31.242) (width 1.4) (layer "F.Cu") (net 1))
 (segment (start 131.572 28.956) (end 131.572 170.434) (width 1.4) (layer "F.Cu") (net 1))
 (segment (start 94.234 170.434) (end 94.234 28.956) (width 1.4) (layer "F.Cu") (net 1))
 (segment (start 110.236 170.434) (end 112.014 170.434) (width 1.4) (layer "F.Cu") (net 1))
 (segment (start 115.57 170.434) (end 115.57 28.956) (width 1.4) (layer "F.Cu") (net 1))
 (segment (start 65.786 170.434) (end 65.786 28.956) (width 1.4) (layer "F.Cu") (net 1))
 (segment (start 99.568 170.434) (end 101.346 170.434) (width 1.4) (layer "F.Cu") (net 1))
 (segment (start 106.68 28.956) (end 106.68 170.434) (width 1.4) (layer "F.Cu") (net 1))
 (segment (start 53.34 28.956) (end 53.34 170.434) (width 1.4) (layer "F.Cu") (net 1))
 (segment (start 101.346 170.434) (end 101.346 28.956) (width 1.4) (layer "F.Cu") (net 1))
 (segment (start 64.008 28.956) (end 64.008 170.434) (width 1.4) (layer "F.Cu") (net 1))
 (segment (start 44.45 28.956) (end 46.228 28.956) (width 1.4) (layer "F.Cu") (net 1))
 (segment (start 58.674 28.956) (end 60.452 28.956) (width 1.4) (layer "F.Cu") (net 1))
 (segment (start 78.232 170.434) (end 80.01 170.434) (width 1.4) (layer "F.Cu") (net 1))
 (segment (start 71.12 170.434) (end 72.898 170.434) (width 1.4) (layer "F.Cu") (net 1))
 (segment (start 154.686 28.956) (end 156.464 28.956) (width 1.4) (layer "F.Cu") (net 1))
 (segment (start 154.686 170.434) (end 154.686 28.956) (width 1.4) (layer "F.Cu") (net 1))
 (segment (start 138.684 170.434) (end 140.462 170.434) (width 1.4) (layer "F.Cu") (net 1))
 (segment (start 113.792 28.956) (end 113.792 170.434) (width 1.4) (layer "F.Cu") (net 1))
 (segment (start 147.574 28.956) (end 149.352 28.956) (width 1.4) (layer "F.Cu") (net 1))
 (segment (start 126.238 170.434) (end 126.238 28.956) (width 1.4) (layer "F.Cu") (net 1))
 (segment (start 24.892 33.02) (end 24.892 162.306) (width 1.4) (layer "F.Cu") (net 1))
 (segment (start 42.672 170.434) (end 44.45 170.434) (width 1.4) (layer "F.Cu") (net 1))
 (segment (start 112.014 28.956) (end 113.792 28.956) (width 1.4) (layer "F.Cu") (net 1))
 (segment (start 166.116 121.285) (end 165.481 120.65) (width 3) (layer "F.Cu") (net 1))
 (segment (start 55.118 170.434) (end 55.118 28.956) (width 1.4) (layer "F.Cu") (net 1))
 (segment (start 67.564 28.956) (end 67.564 170.434) (width 1.4) (layer "F.Cu") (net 1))
 (segment (start 80.01 170.434) (end 80.01 28.956) (width 1.4) (layer "F.Cu") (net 1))
 (segment (start 90.678 170.434) (end 90.678 28.956) (width 1.4) (layer "F.Cu") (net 1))
 (segment (start 165.481 79.375) (end 165.481 89.535) (width 3) (layer "F.Cu") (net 1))
 (segment (start 32.004 28.956) (end 32.004 168.656) (width 1.4) (layer "F.Cu") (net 1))
 (segment (start 151.13 170.434) (end 151.13 28.956) (width 1.4) (layer "F.Cu") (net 1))
 (segment (start 128.016 28.956) (end 128.016 170.434) (width 1.4) (layer "F.Cu") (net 1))
 (segment (start 97.79 28.956) (end 99.568 28.956) (width 1.4) (layer "F.Cu") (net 1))
 (segment (start 39.116 28.956) (end 39.116 170.434) (width 1.4) (layer "F.Cu") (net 1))
 (segment (start 165.481 120.65) (end 165.481 110.49) (width 3) (layer "F.Cu") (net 1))
 (segment (start 72.898 170.434) (end 72.898 28.956) (width 1.4) (layer "F.Cu") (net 1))
 (segment (start 160.782 28.956) (end 165.481 33.655) (width 3) (layer "F.Cu") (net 1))
 (segment (start 78.232 28.956) (end 78.232 170.434) (width 1.4) (layer "F.Cu") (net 1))
 (segment (start 37.338 170.434) (end 37.338 28.956) (width 1.4) (layer "F.Cu") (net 1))
 (segment (start 104.902 170.434) (end 104.902 28.956) (width 1.4) (layer "F.Cu") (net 1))
 (segment (start 166.116 78.74) (end 165.481 79.375) (width 3) (layer "F.Cu") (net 1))
 (segment (start 138.684 28.956) (end 138.684 170.434) (width 1.4) (layer "F.Cu") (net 1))
 (segment (start 136.906 170.434) (end 136.906 28.956) (width 1.4) (layer "F.Cu") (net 1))
 (segment (start 119.126 28.956) (end 120.904 28.956) (width 1.4) (layer "F.Cu") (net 1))
 (segment (start 110.236 28.956) (end 110.236 170.434) (width 1.4) (layer "F.Cu") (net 1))
 (segment (start 140.462 170.434) (end 140.462 28.956) (width 1.4) (layer "F.Cu") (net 1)))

